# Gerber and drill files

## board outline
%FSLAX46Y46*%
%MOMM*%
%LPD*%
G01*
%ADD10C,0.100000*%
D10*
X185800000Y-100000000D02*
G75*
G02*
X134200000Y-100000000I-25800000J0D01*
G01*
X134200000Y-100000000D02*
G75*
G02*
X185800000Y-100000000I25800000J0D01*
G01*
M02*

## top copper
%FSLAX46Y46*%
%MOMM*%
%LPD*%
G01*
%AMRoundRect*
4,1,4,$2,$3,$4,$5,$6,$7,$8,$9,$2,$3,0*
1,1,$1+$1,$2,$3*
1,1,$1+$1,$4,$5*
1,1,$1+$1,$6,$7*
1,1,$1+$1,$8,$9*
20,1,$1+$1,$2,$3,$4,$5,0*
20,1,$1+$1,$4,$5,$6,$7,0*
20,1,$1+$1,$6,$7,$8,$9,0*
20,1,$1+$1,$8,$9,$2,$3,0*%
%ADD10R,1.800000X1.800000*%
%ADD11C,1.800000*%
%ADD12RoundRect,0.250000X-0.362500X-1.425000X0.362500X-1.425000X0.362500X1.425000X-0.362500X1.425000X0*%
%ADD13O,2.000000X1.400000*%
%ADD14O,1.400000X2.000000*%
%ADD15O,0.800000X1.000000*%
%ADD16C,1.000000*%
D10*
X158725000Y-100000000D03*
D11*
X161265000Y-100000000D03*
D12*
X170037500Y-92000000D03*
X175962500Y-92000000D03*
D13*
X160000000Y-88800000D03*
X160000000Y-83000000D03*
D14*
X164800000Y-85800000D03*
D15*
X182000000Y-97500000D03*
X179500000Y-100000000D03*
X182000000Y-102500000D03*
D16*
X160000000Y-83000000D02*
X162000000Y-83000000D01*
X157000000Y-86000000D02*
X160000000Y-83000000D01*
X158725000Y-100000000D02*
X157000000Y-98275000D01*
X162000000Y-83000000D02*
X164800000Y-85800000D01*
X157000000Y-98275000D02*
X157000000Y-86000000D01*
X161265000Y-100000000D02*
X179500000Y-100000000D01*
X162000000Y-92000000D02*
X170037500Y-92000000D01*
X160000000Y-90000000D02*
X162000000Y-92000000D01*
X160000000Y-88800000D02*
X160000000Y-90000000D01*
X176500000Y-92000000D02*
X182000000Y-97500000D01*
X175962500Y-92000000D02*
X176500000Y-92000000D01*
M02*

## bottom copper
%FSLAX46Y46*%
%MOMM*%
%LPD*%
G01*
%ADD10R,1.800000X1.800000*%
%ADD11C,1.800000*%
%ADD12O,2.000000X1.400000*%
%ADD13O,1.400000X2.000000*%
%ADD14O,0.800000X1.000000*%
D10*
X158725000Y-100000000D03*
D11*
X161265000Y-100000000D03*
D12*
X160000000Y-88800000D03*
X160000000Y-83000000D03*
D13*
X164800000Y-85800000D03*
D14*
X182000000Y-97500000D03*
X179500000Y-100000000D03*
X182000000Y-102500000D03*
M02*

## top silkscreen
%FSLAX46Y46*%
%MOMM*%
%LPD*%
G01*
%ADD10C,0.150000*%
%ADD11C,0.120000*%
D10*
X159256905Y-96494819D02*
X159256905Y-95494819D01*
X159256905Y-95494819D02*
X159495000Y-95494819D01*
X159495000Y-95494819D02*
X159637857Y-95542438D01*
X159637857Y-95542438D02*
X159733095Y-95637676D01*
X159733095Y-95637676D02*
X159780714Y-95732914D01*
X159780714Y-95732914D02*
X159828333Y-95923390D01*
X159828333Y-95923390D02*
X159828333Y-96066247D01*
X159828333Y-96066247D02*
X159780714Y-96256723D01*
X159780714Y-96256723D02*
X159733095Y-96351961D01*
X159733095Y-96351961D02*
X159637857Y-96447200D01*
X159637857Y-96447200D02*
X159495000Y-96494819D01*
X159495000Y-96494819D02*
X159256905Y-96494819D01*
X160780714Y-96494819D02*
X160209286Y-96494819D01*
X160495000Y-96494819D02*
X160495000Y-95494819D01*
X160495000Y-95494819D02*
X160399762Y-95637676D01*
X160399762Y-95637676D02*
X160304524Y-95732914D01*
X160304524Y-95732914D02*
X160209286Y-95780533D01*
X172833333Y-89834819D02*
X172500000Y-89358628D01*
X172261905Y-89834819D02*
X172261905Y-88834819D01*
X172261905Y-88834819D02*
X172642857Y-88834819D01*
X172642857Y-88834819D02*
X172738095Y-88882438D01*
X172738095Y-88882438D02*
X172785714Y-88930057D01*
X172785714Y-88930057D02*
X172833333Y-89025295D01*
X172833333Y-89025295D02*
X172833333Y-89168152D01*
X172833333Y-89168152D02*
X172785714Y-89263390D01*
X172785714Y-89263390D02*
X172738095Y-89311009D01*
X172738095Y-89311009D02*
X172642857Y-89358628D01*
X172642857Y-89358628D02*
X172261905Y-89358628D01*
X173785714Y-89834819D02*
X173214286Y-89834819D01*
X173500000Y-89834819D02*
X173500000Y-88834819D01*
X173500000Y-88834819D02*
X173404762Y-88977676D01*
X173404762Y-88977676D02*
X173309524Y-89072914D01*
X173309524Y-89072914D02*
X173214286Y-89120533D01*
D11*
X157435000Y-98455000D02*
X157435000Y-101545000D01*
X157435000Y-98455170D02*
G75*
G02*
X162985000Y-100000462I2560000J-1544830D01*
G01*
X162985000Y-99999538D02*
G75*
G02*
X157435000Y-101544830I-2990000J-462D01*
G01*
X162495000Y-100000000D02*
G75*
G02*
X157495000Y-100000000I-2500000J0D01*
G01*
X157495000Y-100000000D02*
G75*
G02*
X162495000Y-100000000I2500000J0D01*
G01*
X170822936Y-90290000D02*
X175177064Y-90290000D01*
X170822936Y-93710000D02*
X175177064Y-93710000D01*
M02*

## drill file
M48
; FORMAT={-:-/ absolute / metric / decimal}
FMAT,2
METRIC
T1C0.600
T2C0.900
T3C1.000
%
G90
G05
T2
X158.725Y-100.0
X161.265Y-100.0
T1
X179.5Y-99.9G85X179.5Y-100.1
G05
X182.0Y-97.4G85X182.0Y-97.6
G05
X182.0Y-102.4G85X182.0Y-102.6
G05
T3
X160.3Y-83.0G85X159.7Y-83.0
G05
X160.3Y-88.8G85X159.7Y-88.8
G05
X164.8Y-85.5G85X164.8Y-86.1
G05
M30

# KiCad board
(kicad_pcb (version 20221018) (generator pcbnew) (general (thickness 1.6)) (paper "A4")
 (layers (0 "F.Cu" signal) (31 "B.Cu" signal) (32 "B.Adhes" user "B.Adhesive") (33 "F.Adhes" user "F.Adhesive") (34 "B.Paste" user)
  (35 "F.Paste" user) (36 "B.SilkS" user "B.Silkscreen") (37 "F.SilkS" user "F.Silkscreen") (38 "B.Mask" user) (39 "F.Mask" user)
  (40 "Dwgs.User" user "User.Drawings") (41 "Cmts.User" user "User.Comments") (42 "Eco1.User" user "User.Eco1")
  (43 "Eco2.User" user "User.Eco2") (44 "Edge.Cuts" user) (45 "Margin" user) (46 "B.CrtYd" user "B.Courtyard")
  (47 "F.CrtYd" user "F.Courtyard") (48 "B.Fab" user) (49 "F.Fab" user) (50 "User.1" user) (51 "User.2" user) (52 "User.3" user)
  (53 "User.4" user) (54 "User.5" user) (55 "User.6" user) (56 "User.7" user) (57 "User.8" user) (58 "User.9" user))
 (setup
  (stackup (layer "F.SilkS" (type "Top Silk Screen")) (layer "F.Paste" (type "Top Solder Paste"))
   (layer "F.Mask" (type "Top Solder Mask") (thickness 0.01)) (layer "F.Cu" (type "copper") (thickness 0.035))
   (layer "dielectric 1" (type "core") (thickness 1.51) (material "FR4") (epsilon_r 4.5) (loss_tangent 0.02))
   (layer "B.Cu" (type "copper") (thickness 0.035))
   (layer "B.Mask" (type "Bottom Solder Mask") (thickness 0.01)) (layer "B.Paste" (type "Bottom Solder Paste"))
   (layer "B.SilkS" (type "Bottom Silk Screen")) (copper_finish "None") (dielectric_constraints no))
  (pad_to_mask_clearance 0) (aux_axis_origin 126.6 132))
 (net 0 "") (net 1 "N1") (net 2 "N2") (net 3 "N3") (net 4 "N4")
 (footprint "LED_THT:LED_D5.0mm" (layer "F.Cu") (at 158.725 100)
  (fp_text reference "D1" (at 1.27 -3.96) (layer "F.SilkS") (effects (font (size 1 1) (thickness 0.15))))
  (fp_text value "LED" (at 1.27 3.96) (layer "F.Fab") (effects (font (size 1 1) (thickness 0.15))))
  (fp_line (start -1.29 -1.545) (end -1.29 1.545) (stroke (width 0.12) (type solid)) (layer "F.SilkS"))
  (fp_arc (start -1.29 -1.54483) (mid 2.072002 -2.880433) (end 4.26 0.000462) (stroke (width 0.12) (type solid)) (layer "F.SilkS"))
  (fp_arc (start 4.26 -0.000462) (mid 2.072002 2.880433) (end -1.29 1.54483) (stroke (width 0.12) (type solid)) (layer "F.SilkS"))
  (fp_circle (center 1.27 0) (end 3.77 0) (stroke (width 0.12) (type solid)) (fill none) (layer "F.SilkS"))
  (pad "1" thru_hole rect (at 0 0) (size 1.8 1.8) (drill 0.9) (layers "*.Cu" "*.Mask") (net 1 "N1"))
  (pad "2" thru_hole circle (at 2.54 0) (size 1.8 1.8) (drill 0.9) (layers "*.Cu" "*.Mask") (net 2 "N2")))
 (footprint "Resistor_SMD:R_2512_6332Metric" (layer "F.Cu") (at 173 92)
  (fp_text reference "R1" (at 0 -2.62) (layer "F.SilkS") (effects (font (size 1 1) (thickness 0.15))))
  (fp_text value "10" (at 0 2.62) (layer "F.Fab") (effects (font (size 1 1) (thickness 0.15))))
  (fp_line (start -2.177064 -1.71) (end 2.177064 -1.71) (stroke (width 0.12) (type solid)) (layer "F.SilkS"))
  (fp_line (start -2.177064 1.71) (end 2.177064 1.71) (stroke (width 0.12) (type solid)) (layer "F.SilkS"))
  (pad "1" smd roundrect (at -2.9625 0) (size 1.225 3.35) (layers "F.Cu" "F.Paste" "F.Mask") (roundrect_rratio 0.204082) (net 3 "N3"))
  (pad "2" smd roundrect (at 2.9625 0) (size 1.225 3.35) (layers "F.Cu" "F.Paste" "F.Mask") (roundrect_rratio 0.204082) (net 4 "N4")))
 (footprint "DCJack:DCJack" (layer "B.Cu") (at 160 83 -90)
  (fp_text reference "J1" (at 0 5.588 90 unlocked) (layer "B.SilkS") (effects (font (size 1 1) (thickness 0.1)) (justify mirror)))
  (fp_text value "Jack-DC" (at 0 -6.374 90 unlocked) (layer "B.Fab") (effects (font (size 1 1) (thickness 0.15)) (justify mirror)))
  (pad "1" thru_hole oval (at 5.8 0 270) (size 1.4 2) (drill oval 1 1.6) (layers "*.Cu" "*.Mask") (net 3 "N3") (thermal_bridge_angle 45))
  (pad "2" thru_hole oval (at 0 0 270) (size 1.4 2) (drill oval 1 1.6) (layers "*.Cu" "*.Mask") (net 1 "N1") (thermal_bridge_angle 45))
  (pad "2" thru_hole oval (at 2.8 -4.8 270) (size 2 1.4) (drill oval 1.6 1) (layers "*.Cu" "*.Mask") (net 1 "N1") (thermal_bridge_angle 45)))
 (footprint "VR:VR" (layer "B.Cu") (at 182 100 -90)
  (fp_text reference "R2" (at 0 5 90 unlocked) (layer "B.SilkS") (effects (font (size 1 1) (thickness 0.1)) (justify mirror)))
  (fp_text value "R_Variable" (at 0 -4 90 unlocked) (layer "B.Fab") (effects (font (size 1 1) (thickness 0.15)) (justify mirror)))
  (pad "1" thru_hole oval (at -2.5 0 270) (size 1 0.8) (drill oval 0.8 0.6) (layers "*.Cu" "*.Mask") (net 4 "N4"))
  (pad "2" thru_hole oval (at 0 2.5 270) (size 1 0.8) (drill oval 0.8 0.6) (layers "*.Cu" "*.Mask") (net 2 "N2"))
  (pad "3" thru_hole oval (at 2.5 0 270) (size 1 0.8) (drill oval 0.8 0.6) (layers "*.Cu" "*.Mask")))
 (gr_circle (center 160 100) (end 185.8 100) (stroke (width 0.1) (type default)) (fill none) (layer "Edge.Cuts"))
 (segment (start 160 83) (end 162 83) (width 1) (layer "F.Cu") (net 1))
 (segment (start 157 86) (end 160 83) (width 1) (layer "F.Cu") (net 1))
 (segment (start 158.725 100) (end 157 98.275) (width 1) (layer "F.Cu") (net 1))
 (segment (start 162 83) (end 164.8 85.8) (width 1) (layer "F.Cu") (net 1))
 (segment (start 157 98.275) (end 157 86) (width 1) (layer "F.Cu") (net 1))
 (segment (start 161.265 100) (end 179.5 100) (width 1) (layer "F.Cu") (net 2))
 (segment (start 162 92) (end 170.0375 92) (width 1) (layer "F.Cu") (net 3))
 (segment (start 160 90) (end 162 92) (width 1) (layer "F.Cu") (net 3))
 (segment (start 160 88.8) (end 160 90) (width 1) (layer "F.Cu") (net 3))
 (segment (start 176.5 92) (end 182 97.5) (width 1) (layer "F.Cu") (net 4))
 (segment (start 175.9625 92) (end 176.5 92) (width 1) (layer "F.Cu") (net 4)))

